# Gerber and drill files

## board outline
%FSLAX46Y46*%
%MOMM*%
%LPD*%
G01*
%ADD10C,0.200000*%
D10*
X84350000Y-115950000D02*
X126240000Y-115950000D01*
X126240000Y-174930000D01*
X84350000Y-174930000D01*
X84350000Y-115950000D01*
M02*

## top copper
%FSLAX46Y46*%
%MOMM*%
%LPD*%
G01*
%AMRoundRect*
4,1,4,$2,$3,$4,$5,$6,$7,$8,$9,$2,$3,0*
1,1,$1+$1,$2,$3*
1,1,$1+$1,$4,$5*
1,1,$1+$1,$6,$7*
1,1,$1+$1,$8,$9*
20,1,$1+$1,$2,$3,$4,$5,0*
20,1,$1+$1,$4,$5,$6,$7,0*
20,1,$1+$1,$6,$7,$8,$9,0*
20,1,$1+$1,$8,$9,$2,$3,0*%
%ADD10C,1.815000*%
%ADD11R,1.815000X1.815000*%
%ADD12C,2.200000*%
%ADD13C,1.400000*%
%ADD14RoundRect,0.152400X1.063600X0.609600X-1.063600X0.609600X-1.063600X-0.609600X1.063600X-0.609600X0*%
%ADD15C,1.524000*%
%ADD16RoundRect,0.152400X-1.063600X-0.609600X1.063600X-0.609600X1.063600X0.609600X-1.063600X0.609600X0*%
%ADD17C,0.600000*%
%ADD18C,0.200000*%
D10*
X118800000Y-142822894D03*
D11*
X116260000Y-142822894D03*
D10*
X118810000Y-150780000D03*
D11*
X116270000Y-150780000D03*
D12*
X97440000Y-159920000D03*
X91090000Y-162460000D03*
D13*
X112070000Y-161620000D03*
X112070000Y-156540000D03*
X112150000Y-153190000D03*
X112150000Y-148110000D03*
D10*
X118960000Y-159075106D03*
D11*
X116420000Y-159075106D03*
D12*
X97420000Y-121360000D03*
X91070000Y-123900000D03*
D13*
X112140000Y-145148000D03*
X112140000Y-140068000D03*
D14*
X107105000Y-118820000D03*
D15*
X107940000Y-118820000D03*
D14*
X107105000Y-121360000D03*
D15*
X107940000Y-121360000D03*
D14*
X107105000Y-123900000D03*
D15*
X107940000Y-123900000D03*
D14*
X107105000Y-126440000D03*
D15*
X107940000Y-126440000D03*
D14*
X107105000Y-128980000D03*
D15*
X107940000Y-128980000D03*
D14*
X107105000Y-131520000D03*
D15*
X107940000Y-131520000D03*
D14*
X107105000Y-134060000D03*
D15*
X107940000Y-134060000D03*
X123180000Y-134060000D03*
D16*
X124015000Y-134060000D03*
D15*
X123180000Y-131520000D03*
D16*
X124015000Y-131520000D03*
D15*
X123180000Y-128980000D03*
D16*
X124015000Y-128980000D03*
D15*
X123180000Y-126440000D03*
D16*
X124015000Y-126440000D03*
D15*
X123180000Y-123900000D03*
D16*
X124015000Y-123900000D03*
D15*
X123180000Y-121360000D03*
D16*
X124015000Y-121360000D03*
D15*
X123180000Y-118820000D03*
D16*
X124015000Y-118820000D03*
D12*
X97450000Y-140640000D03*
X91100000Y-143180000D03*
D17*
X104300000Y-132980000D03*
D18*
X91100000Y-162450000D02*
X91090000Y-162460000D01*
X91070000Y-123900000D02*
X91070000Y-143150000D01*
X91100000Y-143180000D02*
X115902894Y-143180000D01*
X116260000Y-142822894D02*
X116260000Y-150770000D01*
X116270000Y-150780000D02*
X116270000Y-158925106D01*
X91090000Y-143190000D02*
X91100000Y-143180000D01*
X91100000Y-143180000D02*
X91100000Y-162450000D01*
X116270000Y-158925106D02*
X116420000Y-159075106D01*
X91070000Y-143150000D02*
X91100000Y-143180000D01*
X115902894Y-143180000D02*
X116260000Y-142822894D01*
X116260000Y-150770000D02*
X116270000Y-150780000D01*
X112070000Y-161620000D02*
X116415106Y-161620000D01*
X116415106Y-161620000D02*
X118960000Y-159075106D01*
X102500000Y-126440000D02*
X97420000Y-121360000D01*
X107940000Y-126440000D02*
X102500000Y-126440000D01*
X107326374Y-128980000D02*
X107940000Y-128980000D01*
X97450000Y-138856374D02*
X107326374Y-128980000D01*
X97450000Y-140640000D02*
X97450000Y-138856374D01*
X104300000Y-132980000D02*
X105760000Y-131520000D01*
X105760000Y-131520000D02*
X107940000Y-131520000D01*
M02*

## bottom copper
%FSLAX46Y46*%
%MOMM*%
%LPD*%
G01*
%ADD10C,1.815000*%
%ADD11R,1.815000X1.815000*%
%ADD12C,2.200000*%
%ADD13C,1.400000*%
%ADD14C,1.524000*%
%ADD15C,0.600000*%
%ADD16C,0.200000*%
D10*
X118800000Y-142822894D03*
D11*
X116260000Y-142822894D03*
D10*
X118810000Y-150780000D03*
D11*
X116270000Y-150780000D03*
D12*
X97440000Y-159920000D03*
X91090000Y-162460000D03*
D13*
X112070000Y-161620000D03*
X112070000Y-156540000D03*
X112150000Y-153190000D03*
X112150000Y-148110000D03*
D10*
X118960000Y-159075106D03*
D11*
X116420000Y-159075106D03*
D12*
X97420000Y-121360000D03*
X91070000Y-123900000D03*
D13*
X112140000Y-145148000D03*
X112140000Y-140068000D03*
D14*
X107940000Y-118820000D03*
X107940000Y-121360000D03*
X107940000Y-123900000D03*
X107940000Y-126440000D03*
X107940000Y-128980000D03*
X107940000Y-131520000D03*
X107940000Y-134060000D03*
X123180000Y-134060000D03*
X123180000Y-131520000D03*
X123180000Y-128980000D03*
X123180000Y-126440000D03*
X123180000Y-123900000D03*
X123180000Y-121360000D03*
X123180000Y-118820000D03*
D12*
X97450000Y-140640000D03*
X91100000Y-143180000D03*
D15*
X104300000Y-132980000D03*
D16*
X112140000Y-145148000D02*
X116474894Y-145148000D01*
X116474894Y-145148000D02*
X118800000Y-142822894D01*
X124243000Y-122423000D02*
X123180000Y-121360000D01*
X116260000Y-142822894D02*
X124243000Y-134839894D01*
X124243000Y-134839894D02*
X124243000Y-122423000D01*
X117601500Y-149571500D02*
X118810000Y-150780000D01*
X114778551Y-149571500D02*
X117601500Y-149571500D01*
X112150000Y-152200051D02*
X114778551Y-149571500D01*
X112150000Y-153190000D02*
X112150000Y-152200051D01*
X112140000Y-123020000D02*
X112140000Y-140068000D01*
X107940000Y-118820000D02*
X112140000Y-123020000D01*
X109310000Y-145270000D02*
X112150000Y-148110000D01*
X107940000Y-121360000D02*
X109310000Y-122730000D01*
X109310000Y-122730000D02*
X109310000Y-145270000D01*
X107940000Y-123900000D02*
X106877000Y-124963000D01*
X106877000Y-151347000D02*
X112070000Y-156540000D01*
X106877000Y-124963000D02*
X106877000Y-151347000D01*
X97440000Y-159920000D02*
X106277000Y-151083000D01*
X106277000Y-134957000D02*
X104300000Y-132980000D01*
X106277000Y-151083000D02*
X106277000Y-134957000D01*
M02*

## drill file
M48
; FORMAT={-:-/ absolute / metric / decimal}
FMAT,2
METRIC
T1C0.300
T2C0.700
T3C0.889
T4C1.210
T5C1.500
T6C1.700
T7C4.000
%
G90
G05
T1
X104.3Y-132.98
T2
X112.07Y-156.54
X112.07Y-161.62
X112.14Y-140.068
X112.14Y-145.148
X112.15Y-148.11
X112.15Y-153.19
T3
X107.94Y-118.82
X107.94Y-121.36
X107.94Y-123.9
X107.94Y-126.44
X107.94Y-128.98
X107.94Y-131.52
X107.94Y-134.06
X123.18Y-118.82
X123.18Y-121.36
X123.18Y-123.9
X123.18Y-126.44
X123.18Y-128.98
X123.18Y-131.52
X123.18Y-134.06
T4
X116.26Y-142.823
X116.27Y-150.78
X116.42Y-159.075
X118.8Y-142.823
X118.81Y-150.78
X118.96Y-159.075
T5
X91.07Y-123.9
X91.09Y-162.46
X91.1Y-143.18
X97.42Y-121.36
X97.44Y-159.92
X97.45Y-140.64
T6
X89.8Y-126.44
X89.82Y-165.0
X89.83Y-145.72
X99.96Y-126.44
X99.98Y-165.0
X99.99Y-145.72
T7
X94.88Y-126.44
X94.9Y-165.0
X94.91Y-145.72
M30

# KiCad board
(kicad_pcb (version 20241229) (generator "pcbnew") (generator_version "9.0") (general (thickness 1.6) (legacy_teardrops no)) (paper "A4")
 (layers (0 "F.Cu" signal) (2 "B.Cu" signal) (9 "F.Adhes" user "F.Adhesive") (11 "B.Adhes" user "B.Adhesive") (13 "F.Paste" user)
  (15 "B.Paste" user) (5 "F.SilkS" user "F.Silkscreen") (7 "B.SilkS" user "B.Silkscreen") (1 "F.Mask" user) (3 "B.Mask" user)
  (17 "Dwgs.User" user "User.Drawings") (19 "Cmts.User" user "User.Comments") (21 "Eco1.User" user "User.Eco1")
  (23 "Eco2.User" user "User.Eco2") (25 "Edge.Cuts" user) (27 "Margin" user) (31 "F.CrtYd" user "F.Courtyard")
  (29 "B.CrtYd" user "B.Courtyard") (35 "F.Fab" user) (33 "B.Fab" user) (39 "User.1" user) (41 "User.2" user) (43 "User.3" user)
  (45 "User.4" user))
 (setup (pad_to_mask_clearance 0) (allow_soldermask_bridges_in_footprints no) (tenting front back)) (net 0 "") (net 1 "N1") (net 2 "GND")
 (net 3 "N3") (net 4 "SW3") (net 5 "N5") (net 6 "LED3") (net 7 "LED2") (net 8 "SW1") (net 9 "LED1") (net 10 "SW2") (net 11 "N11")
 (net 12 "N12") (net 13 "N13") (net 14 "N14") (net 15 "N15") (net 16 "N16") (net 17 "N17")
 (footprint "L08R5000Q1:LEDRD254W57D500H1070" (layer "F.Cu") (at 117.53 142.822894)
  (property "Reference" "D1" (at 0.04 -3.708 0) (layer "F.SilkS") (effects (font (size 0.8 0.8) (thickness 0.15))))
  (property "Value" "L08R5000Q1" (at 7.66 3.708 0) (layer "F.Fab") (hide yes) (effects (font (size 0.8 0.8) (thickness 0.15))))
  (pad "A" thru_hole circle (at 1.27 0) (size 1.815 1.815) (drill 1.21) (layers "*.Cu" "*.Mask") (remove_unused_layers no) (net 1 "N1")
   (solder_mask_margin 0.102))
  (pad "C" thru_hole rect (at -1.27 0) (size 1.815 1.815) (drill 1.21) (layers "*.Cu" "*.Mask") (remove_unused_layers no) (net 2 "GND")
   (solder_mask_margin 0.102)))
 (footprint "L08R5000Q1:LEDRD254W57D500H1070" (layer "F.Cu") (at 117.54 150.78)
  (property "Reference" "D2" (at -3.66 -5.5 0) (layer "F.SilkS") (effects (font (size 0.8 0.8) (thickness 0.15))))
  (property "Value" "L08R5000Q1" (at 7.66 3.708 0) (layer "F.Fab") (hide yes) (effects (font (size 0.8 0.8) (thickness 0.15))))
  (pad "A" thru_hole circle (at 1.27 0) (size 1.815 1.815) (drill 1.21) (layers "*.Cu" "*.Mask") (remove_unused_layers no) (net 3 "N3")
   (solder_mask_margin 0.102))
  (pad "C" thru_hole rect (at -1.27 0) (size 1.815 1.815) (drill 1.21) (layers "*.Cu" "*.Mask") (remove_unused_layers no) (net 2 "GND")
   (solder_mask_margin 0.102)))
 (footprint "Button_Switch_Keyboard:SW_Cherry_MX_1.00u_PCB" (layer "F.Cu") (at 97.44 159.92)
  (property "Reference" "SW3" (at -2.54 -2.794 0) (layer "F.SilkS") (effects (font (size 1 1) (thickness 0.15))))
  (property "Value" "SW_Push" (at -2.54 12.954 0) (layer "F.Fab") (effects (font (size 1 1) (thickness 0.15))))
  (pad "" np_thru_hole circle (at -7.62 5.08) (size 1.7 1.7) (drill 1.7) (layers "*.Cu" "*.Mask"))
  (pad "" np_thru_hole circle (at -2.54 5.08) (size 4 4) (drill 4) (layers "*.Cu" "*.Mask"))
  (pad "" np_thru_hole circle (at 2.54 5.08) (size 1.7 1.7) (drill 1.7) (layers "*.Cu" "*.Mask"))
  (pad "1" thru_hole circle (at 0 0) (size 2.2 2.2) (drill 1.5) (layers "*.Cu" "*.Mask") (remove_unused_layers no) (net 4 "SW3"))
  (pad "2" thru_hole circle (at -6.35 2.54) (size 2.2 2.2) (drill 1.5) (layers "*.Cu" "*.Mask") (remove_unused_layers no) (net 2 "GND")))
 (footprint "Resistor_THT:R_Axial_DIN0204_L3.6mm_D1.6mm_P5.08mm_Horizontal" (layer "F.Cu") (at 112.07 161.62 90)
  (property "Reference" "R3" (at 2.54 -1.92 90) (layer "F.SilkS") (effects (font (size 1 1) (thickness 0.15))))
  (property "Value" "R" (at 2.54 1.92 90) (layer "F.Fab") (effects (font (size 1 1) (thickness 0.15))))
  (pad "1" thru_hole circle (at 0 0 90) (size 1.4 1.4) (drill 0.7) (layers "*.Cu" "*.Mask") (remove_unused_layers no) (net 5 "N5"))
  (pad "2" thru_hole circle (at 5.08 0 90) (size 1.4 1.4) (drill 0.7) (layers "*.Cu" "*.Mask") (remove_unused_layers no) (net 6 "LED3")))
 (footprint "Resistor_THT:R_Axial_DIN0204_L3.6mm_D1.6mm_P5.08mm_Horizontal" (layer "F.Cu") (at 112.15 153.19 90)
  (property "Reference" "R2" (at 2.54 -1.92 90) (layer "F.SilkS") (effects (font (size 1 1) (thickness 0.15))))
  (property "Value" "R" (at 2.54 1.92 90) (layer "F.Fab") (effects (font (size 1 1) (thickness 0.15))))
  (pad "1" thru_hole circle (at 0 0 90) (size 1.4 1.4) (drill 0.7) (layers "*.Cu" "*.Mask") (remove_unused_layers no) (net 3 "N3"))
  (pad "2" thru_hole circle (at 5.08 0 90) (size 1.4 1.4) (drill 0.7) (layers "*.Cu" "*.Mask") (remove_unused_layers no) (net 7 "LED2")))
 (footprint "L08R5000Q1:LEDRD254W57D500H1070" (layer "F.Cu") (at 117.69 159.075106)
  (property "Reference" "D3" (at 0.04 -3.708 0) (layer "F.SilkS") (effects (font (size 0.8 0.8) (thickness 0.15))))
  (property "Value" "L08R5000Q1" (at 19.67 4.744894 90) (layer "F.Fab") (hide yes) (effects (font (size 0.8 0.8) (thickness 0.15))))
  (pad "A" thru_hole circle (at 1.27 0) (size 1.815 1.815) (drill 1.21) (layers "*.Cu" "*.Mask") (remove_unused_layers no) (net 5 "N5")
   (solder_mask_margin 0.102))
  (pad "C" thru_hole rect (at -1.27 0) (size 1.815 1.815) (drill 1.21) (layers "*.Cu" "*.Mask") (remove_unused_layers no) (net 2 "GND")
   (solder_mask_margin 0.102)))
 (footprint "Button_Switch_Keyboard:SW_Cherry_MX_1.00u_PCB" (layer "F.Cu") (at 97.42 121.36)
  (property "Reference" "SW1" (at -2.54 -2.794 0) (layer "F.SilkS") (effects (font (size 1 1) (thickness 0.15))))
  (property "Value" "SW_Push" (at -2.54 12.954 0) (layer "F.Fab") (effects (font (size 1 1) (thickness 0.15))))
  (pad "" np_thru_hole circle (at -7.62 5.08) (size 1.7 1.7) (drill 1.7) (layers "*.Cu" "*.Mask"))
  (pad "" np_thru_hole circle (at -2.54 5.08) (size 4 4) (drill 4) (layers "*.Cu" "*.Mask"))
  (pad "" np_thru_hole circle (at 2.54 5.08) (size 1.7 1.7) (drill 1.7) (layers "*.Cu" "*.Mask"))
  (pad "1" thru_hole circle (at 0 0) (size 2.2 2.2) (drill 1.5) (layers "*.Cu" "*.Mask") (remove_unused_layers no) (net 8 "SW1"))
  (pad "2" thru_hole circle (at -6.35 2.54) (size 2.2 2.2) (drill 1.5) (layers "*.Cu" "*.Mask") (remove_unused_layers no) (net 2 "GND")))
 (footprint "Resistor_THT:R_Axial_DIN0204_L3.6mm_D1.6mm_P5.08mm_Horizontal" (layer "F.Cu") (at 112.14 145.148 90)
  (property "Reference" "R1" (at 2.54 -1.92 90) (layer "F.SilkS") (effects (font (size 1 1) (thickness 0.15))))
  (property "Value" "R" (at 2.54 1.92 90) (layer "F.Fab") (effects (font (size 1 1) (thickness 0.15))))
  (pad "1" thru_hole circle (at 0 0 90) (size 1.4 1.4) (drill 0.7) (layers "*.Cu" "*.Mask") (remove_unused_layers no) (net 1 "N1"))
  (pad "2" thru_hole circle (at 5.08 0 90) (size 1.4 1.4) (drill 0.7) (layers "*.Cu" "*.Mask") (remove_unused_layers no) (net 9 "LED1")))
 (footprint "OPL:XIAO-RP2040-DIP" (layer "F.Cu") (at 115.56 126.44)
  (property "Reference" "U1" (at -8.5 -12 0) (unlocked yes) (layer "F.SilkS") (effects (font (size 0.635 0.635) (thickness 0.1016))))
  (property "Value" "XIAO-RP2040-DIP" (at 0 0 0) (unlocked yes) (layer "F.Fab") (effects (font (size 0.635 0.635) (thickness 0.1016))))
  (pad "1" smd roundrect (at -8.455 -7.62 180) (size 2.432 1.524) (layers "F.Cu" "F.Mask") (roundrect_rratio 0.1) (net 9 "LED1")
   (thermal_bridge_angle 45))
  (pad "1" thru_hole circle (at -7.62 -7.62 180) (size 1.524 1.524) (drill 0.889) (layers "*.Cu" "*.Mask") (remove_unused_layers no)
   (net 9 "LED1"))
  (pad "2" smd roundrect (at -8.455 -5.08 180) (size 2.432 1.524) (layers "F.Cu" "F.Mask") (roundrect_rratio 0.1) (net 7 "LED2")
   (thermal_bridge_angle 45))
  (pad "2" thru_hole circle (at -7.62 -5.08 180) (size 1.524 1.524) (drill 0.889) (layers "*.Cu" "*.Mask") (remove_unused_layers no)
   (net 7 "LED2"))
  (pad "3" smd roundrect (at -8.455 -2.54 180) (size 2.432 1.524) (layers "F.Cu" "F.Mask") (roundrect_rratio 0.1) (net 6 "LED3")
   (thermal_bridge_angle 45))
  (pad "3" thru_hole circle (at -7.62 -2.54 180) (size 1.524 1.524) (drill 0.889) (layers "*.Cu" "*.Mask") (remove_unused_layers no)
   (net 6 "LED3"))
  (pad "4" smd roundrect (at -8.455 0 180) (size 2.432 1.524) (layers "F.Cu" "F.Mask") (roundrect_rratio 0.1) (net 8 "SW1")
   (thermal_bridge_angle 45))
  (pad "4" thru_hole circle (at -7.62 0 180) (size 1.524 1.524) (drill 0.889) (layers "*.Cu" "*.Mask") (remove_unused_layers no)
   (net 8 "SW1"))
  (pad "5" smd roundrect (at -8.455 2.54 180) (size 2.432 1.524) (layers "F.Cu" "F.Mask") (roundrect_rratio 0.1) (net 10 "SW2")
   (thermal_bridge_angle 45))
  (pad "5" thru_hole circle (at -7.62 2.54 180) (size 1.524 1.524) (drill 0.889) (layers "*.Cu" "*.Mask") (remove_unused_layers no)
   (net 10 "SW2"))
  (pad "6" smd roundrect (at -8.455 5.08 180) (size 2.432 1.524) (layers "F.Cu" "F.Mask") (roundrect_rratio 0.1) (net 4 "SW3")
   (thermal_bridge_angle 45))
  (pad "6" thru_hole circle (at -7.62 5.08 180) (size 1.524 1.524) (drill 0.889) (layers "*.Cu" "*.Mask") (remove_unused_layers no)
   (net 4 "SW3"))
  (pad "7" smd roundrect (at -8.455 7.62 180) (size 2.432 1.524) (layers "F.Cu" "F.Mask") (roundrect_rratio 0.1) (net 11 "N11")
   (thermal_bridge_angle 45))
  (pad "7" thru_hole circle (at -7.62 7.62 180) (size 1.524 1.524) (drill 0.889) (layers "*.Cu" "*.Mask") (remove_unused_layers no)
   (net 11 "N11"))
  (pad "8" thru_hole circle (at 7.62 7.62) (size 1.524 1.524) (drill 0.889) (layers "*.Cu" "*.Mask") (remove_unused_layers no)
   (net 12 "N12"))
  (pad "8" smd roundrect (at 8.455 7.62) (size 2.432 1.524) (layers "F.Cu" "F.Mask") (roundrect_rratio 0.1) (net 12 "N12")
   (thermal_bridge_angle 45))
  (pad "9" thru_hole circle (at 7.62 5.08) (size 1.524 1.524) (drill 0.889) (layers "*.Cu" "*.Mask") (remove_unused_layers no)
   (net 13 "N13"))
  (pad "9" smd roundrect (at 8.455 5.08) (size 2.432 1.524) (layers "F.Cu" "F.Mask") (roundrect_rratio 0.1) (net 13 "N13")
   (thermal_bridge_angle 45))
  (pad "10" thru_hole circle (at 7.62 2.54) (size 1.524 1.524) (drill 0.889) (layers "*.Cu" "*.Mask") (remove_unused_layers no)
   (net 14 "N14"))
  (pad "10" smd roundrect (at 8.455 2.54) (size 2.432 1.524) (layers "F.Cu" "F.Mask") (roundrect_rratio 0.1) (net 14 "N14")
   (thermal_bridge_angle 45))
  (pad "11" thru_hole circle (at 7.62 0) (size 1.524 1.524) (drill 0.889) (layers "*.Cu" "*.Mask") (remove_unused_layers no) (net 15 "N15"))
  (pad "11" smd roundrect (at 8.455 0) (size 2.432 1.524) (layers "F.Cu" "F.Mask") (roundrect_rratio 0.1) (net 15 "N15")
   (thermal_bridge_angle 45))
  (pad "12" thru_hole circle (at 7.62 -2.54) (size 1.524 1.524) (drill 0.889) (layers "*.Cu" "*.Mask") (remove_unused_layers no)
   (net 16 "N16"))
  (pad "12" smd roundrect (at 8.455 -2.54) (size 2.432 1.524) (layers "F.Cu" "F.Mask") (roundrect_rratio 0.1) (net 16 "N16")
   (thermal_bridge_angle 45))
  (pad "13" thru_hole circle (at 7.62 -5.08) (size 1.524 1.524) (drill 0.889) (layers "*.Cu" "*.Mask") (remove_unused_layers no)
   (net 2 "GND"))
  (pad "13" smd roundrect (at 8.455 -5.08) (size 2.432 1.524) (layers "F.Cu" "F.Mask") (roundrect_rratio 0.1) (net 2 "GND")
   (thermal_bridge_angle 45))
  (pad "14" thru_hole circle (at 7.62 -7.62) (size 1.524 1.524) (drill 0.889) (layers "*.Cu" "*.Mask") (remove_unused_layers no)
   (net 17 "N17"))
  (pad "14" smd roundrect (at 8.455 -7.62) (size 2.432 1.524) (layers "F.Cu" "F.Mask") (roundrect_rratio 0.1) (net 17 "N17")
   (thermal_bridge_angle 45)))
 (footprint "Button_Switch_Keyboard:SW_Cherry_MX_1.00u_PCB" (layer "F.Cu") (at 97.45 140.64)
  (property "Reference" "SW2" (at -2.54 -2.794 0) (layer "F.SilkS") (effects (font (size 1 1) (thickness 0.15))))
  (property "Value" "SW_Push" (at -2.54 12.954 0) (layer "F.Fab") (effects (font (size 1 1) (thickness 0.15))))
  (pad "" np_thru_hole circle (at -7.62 5.08) (size 1.7 1.7) (drill 1.7) (layers "*.Cu" "*.Mask"))
  (pad "" np_thru_hole circle (at -2.54 5.08) (size 4 4) (drill 4) (layers "*.Cu" "*.Mask"))
  (pad "" np_thru_hole circle (at 2.54 5.08) (size 1.7 1.7) (drill 1.7) (layers "*.Cu" "*.Mask"))
  (pad "1" thru_hole circle (at 0 0) (size 2.2 2.2) (drill 1.5) (layers "*.Cu" "*.Mask") (remove_unused_layers no) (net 10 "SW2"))
  (pad "2" thru_hole circle (at -6.35 2.54) (size 2.2 2.2) (drill 1.5) (layers "*.Cu" "*.Mask") (remove_unused_layers no) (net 2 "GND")))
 (gr_rect (start 84.35 115.95) (end 126.24 174.93) (stroke (width 0.2) (type solid)) (fill no) (layer "Edge.Cuts"))
 (segment (start 112.14 145.148) (end 116.474894 145.148) (width 0.2) (layer "B.Cu") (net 1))
 (segment (start 116.474894 145.148) (end 118.8 142.822894) (width 0.2) (layer "B.Cu") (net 1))
 (segment (start 91.1 162.45) (end 91.09 162.46) (width 0.2) (layer "F.Cu") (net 2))
 (segment (start 91.07 123.9) (end 91.07 143.15) (width 0.2) (layer "F.Cu") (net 2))
 (segment (start 91.1 143.18) (end 115.902894 143.18) (width 0.2) (layer "F.Cu") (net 2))
 (segment (start 116.26 142.822894) (end 116.26 150.77) (width 0.2) (layer "F.Cu") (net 2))
 (segment (start 116.27 150.78) (end 116.27 158.925106) (width 0.2) (layer "F.Cu") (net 2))
 (segment (start 91.09 143.19) (end 91.1 143.18) (width 0.2) (layer "F.Cu") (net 2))
 (segment (start 91.1 143.18) (end 91.1 162.45) (width 0.2) (layer "F.Cu") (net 2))
 (segment (start 116.27 158.925106) (end 116.42 159.075106) (width 0.2) (layer "F.Cu") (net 2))
 (segment (start 91.07 143.15) (end 91.1 143.18) (width 0.2) (layer "F.Cu") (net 2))
 (segment (start 115.902894 143.18) (end 116.26 142.822894) (width 0.2) (layer "F.Cu") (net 2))
 (segment (start 116.26 150.77) (end 116.27 150.78) (width 0.2) (layer "F.Cu") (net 2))
 (segment (start 124.243 122.423) (end 123.18 121.36) (width 0.2) (layer "B.Cu") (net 2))
 (segment (start 116.26 142.822894) (end 124.243 134.839894) (width 0.2) (layer "B.Cu") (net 2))
 (segment (start 124.243 134.839894) (end 124.243 122.423) (width 0.2) (layer "B.Cu") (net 2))
 (segment (start 117.6015 149.5715) (end 118.81 150.78) (width 0.2) (layer "B.Cu") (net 3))
 (segment (start 114.778551 149.5715) (end 117.6015 149.5715) (width 0.2) (layer "B.Cu") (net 3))
 (segment (start 112.15 152.200051) (end 114.778551 149.5715) (width 0.2) (layer "B.Cu") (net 3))
 (segment (start 112.15 153.19) (end 112.15 152.200051) (width 0.2) (layer "B.Cu") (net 3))
 (segment (start 112.07 161.62) (end 116.415106 161.62) (width 0.2) (layer "F.Cu") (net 5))
 (segment (start 116.415106 161.62) (end 118.96 159.075106) (width 0.2) (layer "F.Cu") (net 5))
 (segment (start 112.14 123.02) (end 112.14 140.068) (width 0.2) (layer "B.Cu") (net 9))
 (segment (start 107.94 118.82) (end 112.14 123.02) (width 0.2) (layer "B.Cu") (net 9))
 (segment (start 109.31 145.27) (end 112.15 148.11) (width 0.2) (layer "B.Cu") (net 7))
 (segment (start 107.94 121.36) (end 109.31 122.73) (width 0.2) (layer "B.Cu") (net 7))
 (segment (start 109.31 122.73) (end 109.31 145.27) (width 0.2) (layer "B.Cu") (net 7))
 (segment (start 107.94 123.9) (end 106.877 124.963) (width 0.2) (layer "B.Cu") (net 6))
 (segment (start 106.877 151.347) (end 112.07 156.54) (width 0.2) (layer "B.Cu") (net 6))
 (segment (start 106.877 124.963) (end 106.877 151.347) (width 0.2) (layer "B.Cu") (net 6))
 (segment (start 102.5 126.44) (end 97.42 121.36) (width 0.2) (layer "F.Cu") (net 8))
 (segment (start 107.94 126.44) (end 102.5 126.44) (width 0.2) (layer "F.Cu") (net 8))
 (segment (start 107.326374 128.98) (end 107.94 128.98) (width 0.2) (layer "F.Cu") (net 10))
 (segment (start 97.45 138.856374) (end 107.326374 128.98) (width 0.2) (layer "F.Cu") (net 10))
 (segment (start 97.45 140.64) (end 97.45 138.856374) (width 0.2) (layer "F.Cu") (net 10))
 (segment (start 104.3 132.98) (end 105.76 131.52) (width 0.2) (layer "F.Cu") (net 4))
 (segment (start 105.76 131.52) (end 107.94 131.52) (width 0.2) (layer "F.Cu") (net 4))
 (via (at 104.3 132.98) (size 0.6) (drill 0.3) (layers "F.Cu" "B.Cu") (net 4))
 (segment (start 97.44 159.92) (end 106.277 151.083) (width 0.2) (layer "B.Cu") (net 4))
 (segment (start 106.277 134.957) (end 104.3 132.98) (width 0.2) (layer "B.Cu") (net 4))
 (segment (start 106.277 151.083) (end 106.277 134.957) (width 0.2) (layer "B.Cu") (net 4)))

